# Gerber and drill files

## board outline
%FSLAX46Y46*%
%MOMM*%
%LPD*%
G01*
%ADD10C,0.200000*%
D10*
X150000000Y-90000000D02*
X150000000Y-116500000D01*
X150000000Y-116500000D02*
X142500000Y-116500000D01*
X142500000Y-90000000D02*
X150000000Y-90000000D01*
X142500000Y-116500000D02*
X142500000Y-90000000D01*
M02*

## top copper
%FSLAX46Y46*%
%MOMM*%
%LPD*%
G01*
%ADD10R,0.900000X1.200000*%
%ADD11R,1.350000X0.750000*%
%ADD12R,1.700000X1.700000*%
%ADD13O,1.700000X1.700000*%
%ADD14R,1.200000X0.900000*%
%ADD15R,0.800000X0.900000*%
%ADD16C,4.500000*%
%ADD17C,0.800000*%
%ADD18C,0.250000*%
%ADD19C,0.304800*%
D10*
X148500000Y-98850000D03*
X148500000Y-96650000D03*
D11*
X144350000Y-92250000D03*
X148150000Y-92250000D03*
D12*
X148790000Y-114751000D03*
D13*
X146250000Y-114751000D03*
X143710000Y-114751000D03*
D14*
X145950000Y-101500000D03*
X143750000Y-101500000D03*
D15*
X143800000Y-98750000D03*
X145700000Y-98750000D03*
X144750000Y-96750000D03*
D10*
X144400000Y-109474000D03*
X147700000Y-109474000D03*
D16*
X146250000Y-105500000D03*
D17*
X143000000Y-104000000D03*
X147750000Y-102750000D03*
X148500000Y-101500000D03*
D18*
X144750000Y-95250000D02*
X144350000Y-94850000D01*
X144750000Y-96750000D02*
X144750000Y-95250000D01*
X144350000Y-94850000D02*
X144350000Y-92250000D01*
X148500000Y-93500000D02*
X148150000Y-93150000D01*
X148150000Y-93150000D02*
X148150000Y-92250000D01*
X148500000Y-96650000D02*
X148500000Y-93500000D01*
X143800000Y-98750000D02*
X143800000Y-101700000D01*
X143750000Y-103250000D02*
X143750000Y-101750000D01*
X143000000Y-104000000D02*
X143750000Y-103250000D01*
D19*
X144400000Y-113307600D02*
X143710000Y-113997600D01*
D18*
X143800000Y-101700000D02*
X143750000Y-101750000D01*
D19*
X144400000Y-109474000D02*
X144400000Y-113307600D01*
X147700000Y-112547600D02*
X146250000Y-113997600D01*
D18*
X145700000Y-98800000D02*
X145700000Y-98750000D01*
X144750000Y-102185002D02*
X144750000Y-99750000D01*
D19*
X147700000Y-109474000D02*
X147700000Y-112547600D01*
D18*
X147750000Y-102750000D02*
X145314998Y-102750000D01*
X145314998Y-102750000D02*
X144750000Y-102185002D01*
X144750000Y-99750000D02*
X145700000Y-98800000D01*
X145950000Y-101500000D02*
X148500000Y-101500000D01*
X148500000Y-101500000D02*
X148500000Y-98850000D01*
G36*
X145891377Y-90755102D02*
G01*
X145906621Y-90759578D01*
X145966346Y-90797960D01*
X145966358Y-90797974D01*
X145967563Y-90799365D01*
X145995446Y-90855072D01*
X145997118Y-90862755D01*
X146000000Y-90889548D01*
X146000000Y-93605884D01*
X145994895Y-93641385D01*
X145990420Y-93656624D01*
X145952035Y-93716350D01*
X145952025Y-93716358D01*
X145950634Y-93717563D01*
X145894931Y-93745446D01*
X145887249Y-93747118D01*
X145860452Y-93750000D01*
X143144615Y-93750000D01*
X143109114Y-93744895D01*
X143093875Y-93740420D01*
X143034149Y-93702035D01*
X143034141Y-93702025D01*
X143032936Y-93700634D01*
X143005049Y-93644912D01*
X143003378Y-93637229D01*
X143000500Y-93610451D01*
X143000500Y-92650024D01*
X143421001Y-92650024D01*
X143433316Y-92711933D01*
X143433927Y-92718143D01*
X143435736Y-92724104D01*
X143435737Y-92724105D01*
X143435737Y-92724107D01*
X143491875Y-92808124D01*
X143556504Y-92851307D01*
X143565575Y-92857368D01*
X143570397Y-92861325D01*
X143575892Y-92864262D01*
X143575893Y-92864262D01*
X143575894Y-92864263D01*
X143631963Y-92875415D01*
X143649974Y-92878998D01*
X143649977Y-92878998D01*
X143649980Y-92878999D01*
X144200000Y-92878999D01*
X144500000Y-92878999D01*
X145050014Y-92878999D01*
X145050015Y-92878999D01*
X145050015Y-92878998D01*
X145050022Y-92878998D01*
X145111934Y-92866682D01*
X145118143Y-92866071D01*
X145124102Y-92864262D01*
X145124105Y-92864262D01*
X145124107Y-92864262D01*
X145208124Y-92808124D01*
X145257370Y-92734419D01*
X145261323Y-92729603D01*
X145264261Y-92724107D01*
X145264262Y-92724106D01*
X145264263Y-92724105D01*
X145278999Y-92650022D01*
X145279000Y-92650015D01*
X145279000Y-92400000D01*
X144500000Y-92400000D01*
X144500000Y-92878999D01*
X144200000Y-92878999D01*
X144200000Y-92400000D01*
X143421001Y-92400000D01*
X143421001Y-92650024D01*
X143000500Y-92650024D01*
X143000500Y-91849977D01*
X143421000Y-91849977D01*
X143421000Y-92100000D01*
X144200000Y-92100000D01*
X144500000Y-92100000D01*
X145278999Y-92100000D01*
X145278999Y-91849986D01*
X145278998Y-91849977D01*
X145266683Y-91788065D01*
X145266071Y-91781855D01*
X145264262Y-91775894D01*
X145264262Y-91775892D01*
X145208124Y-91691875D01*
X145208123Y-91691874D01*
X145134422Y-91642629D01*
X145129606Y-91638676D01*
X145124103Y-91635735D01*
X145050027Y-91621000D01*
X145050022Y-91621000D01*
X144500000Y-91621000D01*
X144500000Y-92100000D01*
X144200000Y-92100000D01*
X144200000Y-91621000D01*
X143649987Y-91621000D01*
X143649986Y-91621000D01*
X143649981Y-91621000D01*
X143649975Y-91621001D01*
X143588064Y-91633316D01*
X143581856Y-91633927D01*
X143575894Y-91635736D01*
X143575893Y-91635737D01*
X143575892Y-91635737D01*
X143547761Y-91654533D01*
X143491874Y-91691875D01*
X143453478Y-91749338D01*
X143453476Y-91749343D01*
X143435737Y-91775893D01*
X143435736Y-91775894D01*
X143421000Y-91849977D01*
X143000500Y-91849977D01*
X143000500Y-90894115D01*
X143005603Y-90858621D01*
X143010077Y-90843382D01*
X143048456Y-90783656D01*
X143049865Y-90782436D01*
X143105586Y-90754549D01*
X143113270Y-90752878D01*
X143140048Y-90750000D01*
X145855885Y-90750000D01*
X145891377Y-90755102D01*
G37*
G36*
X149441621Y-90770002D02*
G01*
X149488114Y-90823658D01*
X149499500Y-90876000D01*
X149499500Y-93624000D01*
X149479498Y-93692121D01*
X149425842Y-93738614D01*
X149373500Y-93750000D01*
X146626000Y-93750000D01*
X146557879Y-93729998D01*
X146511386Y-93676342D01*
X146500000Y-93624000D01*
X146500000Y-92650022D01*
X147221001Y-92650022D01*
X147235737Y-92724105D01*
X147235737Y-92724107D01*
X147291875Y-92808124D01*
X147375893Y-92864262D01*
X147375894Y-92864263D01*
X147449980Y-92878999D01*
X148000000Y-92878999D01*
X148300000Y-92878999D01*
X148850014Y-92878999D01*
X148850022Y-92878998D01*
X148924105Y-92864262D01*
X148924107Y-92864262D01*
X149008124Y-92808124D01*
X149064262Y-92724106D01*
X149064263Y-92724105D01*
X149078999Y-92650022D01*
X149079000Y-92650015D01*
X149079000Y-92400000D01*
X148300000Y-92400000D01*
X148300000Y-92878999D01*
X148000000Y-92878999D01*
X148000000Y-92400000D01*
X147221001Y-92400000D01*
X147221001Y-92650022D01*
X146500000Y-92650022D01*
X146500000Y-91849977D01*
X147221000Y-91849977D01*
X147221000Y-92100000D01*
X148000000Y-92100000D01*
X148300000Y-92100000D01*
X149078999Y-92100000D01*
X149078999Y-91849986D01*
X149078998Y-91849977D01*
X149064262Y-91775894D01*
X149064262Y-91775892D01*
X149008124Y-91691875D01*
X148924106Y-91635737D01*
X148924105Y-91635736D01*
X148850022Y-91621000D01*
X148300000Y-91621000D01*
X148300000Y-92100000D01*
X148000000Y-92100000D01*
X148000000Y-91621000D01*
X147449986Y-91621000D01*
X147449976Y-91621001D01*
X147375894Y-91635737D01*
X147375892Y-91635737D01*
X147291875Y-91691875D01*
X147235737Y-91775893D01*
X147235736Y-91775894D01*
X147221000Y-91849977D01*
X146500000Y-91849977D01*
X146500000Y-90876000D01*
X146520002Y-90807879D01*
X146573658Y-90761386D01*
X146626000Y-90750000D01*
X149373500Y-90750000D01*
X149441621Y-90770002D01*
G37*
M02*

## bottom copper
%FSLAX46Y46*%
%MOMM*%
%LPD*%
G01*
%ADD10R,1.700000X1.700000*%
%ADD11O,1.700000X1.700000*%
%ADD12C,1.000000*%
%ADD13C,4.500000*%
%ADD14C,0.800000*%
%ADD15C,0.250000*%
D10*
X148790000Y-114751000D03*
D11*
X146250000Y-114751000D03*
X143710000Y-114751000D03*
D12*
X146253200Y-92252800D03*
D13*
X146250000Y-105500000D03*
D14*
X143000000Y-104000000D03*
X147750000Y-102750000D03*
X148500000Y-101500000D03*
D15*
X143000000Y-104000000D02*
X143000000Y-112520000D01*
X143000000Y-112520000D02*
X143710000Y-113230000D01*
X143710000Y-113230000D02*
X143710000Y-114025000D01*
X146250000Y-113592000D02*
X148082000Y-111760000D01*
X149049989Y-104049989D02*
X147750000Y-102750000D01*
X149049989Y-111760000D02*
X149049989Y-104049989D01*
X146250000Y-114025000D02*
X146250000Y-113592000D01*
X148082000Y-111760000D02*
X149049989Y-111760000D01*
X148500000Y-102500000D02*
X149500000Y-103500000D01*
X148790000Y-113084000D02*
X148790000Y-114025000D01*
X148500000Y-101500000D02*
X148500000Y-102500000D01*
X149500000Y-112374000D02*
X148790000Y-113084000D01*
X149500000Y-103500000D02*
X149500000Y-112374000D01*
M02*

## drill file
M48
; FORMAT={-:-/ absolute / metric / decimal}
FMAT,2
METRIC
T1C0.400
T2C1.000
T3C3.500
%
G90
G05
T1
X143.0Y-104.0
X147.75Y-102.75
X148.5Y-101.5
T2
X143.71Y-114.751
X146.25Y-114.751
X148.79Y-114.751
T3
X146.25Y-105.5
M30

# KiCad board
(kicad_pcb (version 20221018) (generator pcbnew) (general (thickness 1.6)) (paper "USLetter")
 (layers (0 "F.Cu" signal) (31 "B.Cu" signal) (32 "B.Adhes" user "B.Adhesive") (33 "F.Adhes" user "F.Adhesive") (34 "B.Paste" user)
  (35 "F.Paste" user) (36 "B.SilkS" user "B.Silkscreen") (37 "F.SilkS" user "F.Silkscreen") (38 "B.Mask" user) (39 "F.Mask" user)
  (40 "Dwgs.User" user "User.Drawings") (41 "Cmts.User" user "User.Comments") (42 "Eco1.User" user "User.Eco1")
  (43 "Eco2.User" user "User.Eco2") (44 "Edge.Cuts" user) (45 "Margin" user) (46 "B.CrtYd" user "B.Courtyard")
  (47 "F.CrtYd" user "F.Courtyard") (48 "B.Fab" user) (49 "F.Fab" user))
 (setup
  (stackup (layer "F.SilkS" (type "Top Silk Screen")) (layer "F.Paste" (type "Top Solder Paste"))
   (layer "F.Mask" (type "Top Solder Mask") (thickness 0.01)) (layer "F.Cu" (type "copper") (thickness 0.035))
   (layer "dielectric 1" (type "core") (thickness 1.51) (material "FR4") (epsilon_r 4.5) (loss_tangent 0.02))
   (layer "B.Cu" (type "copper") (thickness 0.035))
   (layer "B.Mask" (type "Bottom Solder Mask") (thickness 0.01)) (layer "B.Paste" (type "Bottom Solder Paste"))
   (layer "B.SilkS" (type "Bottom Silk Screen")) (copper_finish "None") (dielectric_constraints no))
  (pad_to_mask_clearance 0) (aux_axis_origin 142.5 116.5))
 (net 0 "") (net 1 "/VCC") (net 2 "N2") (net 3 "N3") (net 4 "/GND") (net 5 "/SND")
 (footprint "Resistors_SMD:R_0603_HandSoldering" (layer "F.Cu") (at 148.5 97.75 90)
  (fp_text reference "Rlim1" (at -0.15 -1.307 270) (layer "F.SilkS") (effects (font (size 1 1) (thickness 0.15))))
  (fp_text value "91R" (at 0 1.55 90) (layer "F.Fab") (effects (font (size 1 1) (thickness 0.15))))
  (pad "1" smd rect (at -1.1 0 90) (size 1.2 0.9) (layers "F.Cu" "F.Paste" "F.Mask") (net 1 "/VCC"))
  (pad "2" smd rect (at 1.1 0 90) (size 1.2 0.9) (layers "F.Cu" "F.Paste" "F.Mask") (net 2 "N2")))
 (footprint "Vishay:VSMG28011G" (layer "F.Cu") (at 146.25 92.25)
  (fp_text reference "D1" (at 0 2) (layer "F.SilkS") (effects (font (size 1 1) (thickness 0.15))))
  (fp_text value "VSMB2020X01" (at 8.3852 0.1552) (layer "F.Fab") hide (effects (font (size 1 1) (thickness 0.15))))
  (pad "1" smd rect (at -1.9 0) (size 1.35 0.75) (layers "F.Cu" "F.Paste" "F.Mask") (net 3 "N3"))
  (pad "2" smd rect (at 1.9 0) (size 1.35 0.75) (layers "F.Cu" "F.Paste" "F.Mask") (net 2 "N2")))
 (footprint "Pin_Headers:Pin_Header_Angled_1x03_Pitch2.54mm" (layer "F.Cu") (at 148.79 114.751 -90)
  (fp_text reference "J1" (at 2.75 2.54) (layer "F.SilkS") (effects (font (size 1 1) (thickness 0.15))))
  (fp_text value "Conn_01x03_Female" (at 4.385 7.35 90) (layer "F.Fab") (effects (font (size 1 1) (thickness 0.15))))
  (pad "1" thru_hole rect (at 0 0 270) (size 1.7 1.7) (drill 1) (layers "*.Cu" "*.Mask") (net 1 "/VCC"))
  (pad "2" thru_hole oval (at 0 2.54 270) (size 1.7 1.7) (drill 1) (layers "*.Cu" "*.Mask") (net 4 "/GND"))
  (pad "3" thru_hole oval (at 0 5.08 270) (size 1.7 1.7) (drill 1) (layers "*.Cu" "*.Mask") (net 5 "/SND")))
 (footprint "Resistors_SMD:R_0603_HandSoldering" (layer "F.Cu") (at 144.85 101.5 180)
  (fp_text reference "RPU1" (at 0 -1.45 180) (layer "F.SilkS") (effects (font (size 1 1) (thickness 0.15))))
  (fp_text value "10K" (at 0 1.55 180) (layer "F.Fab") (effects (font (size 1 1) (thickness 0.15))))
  (pad "1" smd rect (at -1.1 0 180) (size 1.2 0.9) (layers "F.Cu" "F.Paste" "F.Mask") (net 1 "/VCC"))
  (pad "2" smd rect (at 1.1 0 180) (size 1.2 0.9) (layers "F.Cu" "F.Paste" "F.Mask") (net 5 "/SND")))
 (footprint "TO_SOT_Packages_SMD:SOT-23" (layer "F.Cu") (at 144.75 97.75 90)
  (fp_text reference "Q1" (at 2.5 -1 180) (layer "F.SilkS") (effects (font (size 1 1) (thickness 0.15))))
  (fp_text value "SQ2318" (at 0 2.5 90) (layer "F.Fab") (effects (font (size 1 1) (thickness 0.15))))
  (pad "1" smd rect (at -1 -0.95 90) (size 0.9 0.8) (layers "F.Cu" "F.Paste" "F.Mask") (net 5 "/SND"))
  (pad "2" smd rect (at -1 0.95 90) (size 0.9 0.8) (layers "F.Cu" "F.Paste" "F.Mask") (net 4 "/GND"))
  (pad "3" smd rect (at 1 0 90) (size 0.9 0.8) (layers "F.Cu" "F.Paste" "F.Mask") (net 3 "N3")))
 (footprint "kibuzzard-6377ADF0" (layer "F.Cu") (at 147.574 112.395 90)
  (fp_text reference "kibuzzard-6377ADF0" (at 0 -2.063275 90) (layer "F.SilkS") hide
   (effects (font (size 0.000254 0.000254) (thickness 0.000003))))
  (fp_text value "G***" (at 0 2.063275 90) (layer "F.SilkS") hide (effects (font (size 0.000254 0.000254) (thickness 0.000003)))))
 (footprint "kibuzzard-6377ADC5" (layer "F.Cu") (at 144.018 112.014 90)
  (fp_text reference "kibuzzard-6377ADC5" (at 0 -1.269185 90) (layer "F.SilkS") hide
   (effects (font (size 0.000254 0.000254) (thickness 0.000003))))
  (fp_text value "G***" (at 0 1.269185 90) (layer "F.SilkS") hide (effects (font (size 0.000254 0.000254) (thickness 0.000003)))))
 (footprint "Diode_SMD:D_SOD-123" (layer "F.Cu") (at 146.05 109.474)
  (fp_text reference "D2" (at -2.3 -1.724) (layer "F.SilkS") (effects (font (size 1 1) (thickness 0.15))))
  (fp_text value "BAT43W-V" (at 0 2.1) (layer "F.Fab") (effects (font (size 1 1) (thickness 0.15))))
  (pad "1" smd rect (at -1.65 0) (size 0.9 1.2) (layers "F.Cu" "F.Paste" "F.Mask") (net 5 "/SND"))
  (pad "2" smd rect (at 1.65 0) (size 0.9 1.2) (layers "F.Cu" "F.Paste" "F.Mask") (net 4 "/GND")))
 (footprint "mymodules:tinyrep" (layer "B.Cu") (at 148.717 97.663 90)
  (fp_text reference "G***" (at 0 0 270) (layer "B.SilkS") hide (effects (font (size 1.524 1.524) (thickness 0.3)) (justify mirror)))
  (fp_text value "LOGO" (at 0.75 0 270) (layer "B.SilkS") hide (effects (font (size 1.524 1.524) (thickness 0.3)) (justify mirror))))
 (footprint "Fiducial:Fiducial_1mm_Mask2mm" (layer "B.Cu") (at 146.2532 92.2528 180)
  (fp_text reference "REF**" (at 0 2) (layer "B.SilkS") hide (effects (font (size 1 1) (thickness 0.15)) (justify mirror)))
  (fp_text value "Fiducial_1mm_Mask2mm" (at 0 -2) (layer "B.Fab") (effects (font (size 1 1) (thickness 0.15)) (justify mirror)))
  (pad "" smd circle (at 0 0 180) (size 1 1) (layers "B.Cu" "B.Mask") (solder_mask_margin 0.5) (clearance 0.5)))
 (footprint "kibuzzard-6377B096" (layer "B.Cu") (at 147.574 112.395 -90)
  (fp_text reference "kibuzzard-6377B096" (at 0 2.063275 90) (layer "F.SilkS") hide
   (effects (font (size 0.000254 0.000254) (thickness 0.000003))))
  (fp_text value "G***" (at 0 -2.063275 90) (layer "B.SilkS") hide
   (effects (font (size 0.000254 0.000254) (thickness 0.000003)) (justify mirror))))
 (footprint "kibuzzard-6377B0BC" (layer "B.Cu") (at 144.018 112.014 90)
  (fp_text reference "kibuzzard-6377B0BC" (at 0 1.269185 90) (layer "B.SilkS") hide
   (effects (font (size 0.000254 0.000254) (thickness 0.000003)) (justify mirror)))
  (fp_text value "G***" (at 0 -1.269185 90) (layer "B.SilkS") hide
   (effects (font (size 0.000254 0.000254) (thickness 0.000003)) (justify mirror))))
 (gr_line (start 150 90) (end 150 116.5) (stroke (width 0.2) (type solid)) (layer "Edge.Cuts"))
 (gr_line (start 150 116.5) (end 142.5 116.5) (stroke (width 0.2) (type solid)) (layer "Edge.Cuts"))
 (gr_line (start 142.5 90) (end 150 90) (stroke (width 0.2) (type solid)) (layer "Edge.Cuts"))
 (gr_line (start 142.5 116.5) (end 142.5 90) (stroke (width 0.2) (type solid)) (layer "Edge.Cuts"))
 (via (at 146.25 105.5) (size 4.5) (drill 3.5) (layers "F.Cu" "B.Cu") (free) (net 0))
 (segment (start 144.75 95.25) (end 144.35 94.85) (width 0.25) (layer "F.Cu") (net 3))
 (segment (start 144.75 96.75) (end 144.75 95.25) (width 0.25) (layer "F.Cu") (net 3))
 (segment (start 144.35 94.85) (end 144.35 92.25) (width 0.25) (layer "F.Cu") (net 3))
 (segment (start 148.5 93.5) (end 148.15 93.15) (width 0.25) (layer "F.Cu") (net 2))
 (segment (start 148.15 93.15) (end 148.15 92.25) (width 0.25) (layer "F.Cu") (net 2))
 (segment (start 148.5 96.65) (end 148.5 93.5) (width 0.25) (layer "F.Cu") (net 2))
 (segment (start 143.8 98.75) (end 143.8 101.7) (width 0.25) (layer "F.Cu") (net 5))
 (segment (start 143.75 103.25) (end 143.75 101.75) (width 0.25) (layer "F.Cu") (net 5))
 (segment (start 143 104) (end 143.75 103.25) (width 0.25) (layer "F.Cu") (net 5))
 (segment (start 144.4 113.3076) (end 143.71 113.9976) (width 0.3048) (layer "F.Cu") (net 5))
 (segment (start 143.8 101.7) (end 143.75 101.75) (width 0.25) (layer "F.Cu") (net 5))
 (segment (start 144.4 109.474) (end 144.4 113.3076) (width 0.3048) (layer "F.Cu") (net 5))
 (via (at 143 104) (size 0.8) (drill 0.4) (layers "F.Cu" "B.Cu") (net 5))
 (segment (start 143 104) (end 143 112.52) (width 0.25) (layer "B.Cu") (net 5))
 (segment (start 143 112.52) (end 143.71 113.23) (width 0.25) (layer "B.Cu") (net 5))
 (segment (start 143.71 113.23) (end 143.71 114.025) (width 0.25) (layer "B.Cu") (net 5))
 (segment (start 147.7 112.5476) (end 146.25 113.9976) (width 0.3048) (layer "F.Cu") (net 4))
 (segment (start 145.7 98.8) (end 145.7 98.75) (width 0.25) (layer "F.Cu") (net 4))
 (segment (start 144.75 102.185002) (end 144.75 99.75) (width 0.25) (layer "F.Cu") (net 4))
 (segment (start 147.7 109.474) (end 147.7 112.5476) (width 0.3048) (layer "F.Cu") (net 4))
 (segment (start 147.75 102.75) (end 145.314998 102.75) (width 0.25) (layer "F.Cu") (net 4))
 (segment (start 145.314998 102.75) (end 144.75 102.185002) (width 0.25) (layer "F.Cu") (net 4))
 (segment (start 144.75 99.75) (end 145.7 98.8) (width 0.25) (layer "F.Cu") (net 4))
 (via (at 147.75 102.75) (size 0.8) (drill 0.4) (layers "F.Cu" "B.Cu") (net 4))
 (segment (start 146.25 113.592) (end 148.082 111.76) (width 0.25) (layer "B.Cu") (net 4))
 (segment (start 149.049989 104.049989) (end 147.75 102.75) (width 0.25) (layer "B.Cu") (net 4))
 (segment (start 149.049989 111.76) (end 149.049989 104.049989) (width 0.25) (layer "B.Cu") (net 4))
 (segment (start 146.25 114.025) (end 146.25 113.592) (width 0.25) (layer "B.Cu") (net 4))
 (segment (start 148.082 111.76) (end 149.049989 111.76) (width 0.25) (layer "B.Cu") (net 4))
 (segment (start 145.95 101.5) (end 148.5 101.5) (width 0.25) (layer "F.Cu") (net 1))
 (segment (start 148.5 101.5) (end 148.5 98.85) (width 0.25) (layer "F.Cu") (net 1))
 (via (at 148.5 101.5) (size 0.8) (drill 0.4) (layers "F.Cu" "B.Cu") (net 1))
 (segment (start 148.5 102.5) (end 149.5 103.5) (width 0.25) (layer "B.Cu") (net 1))
 (segment (start 148.79 113.084) (end 148.79 114.025) (width 0.25) (layer "B.Cu") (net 1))
 (segment (start 148.5 101.5) (end 148.5 102.5) (width 0.25) (layer "B.Cu") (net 1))
 (segment (start 149.5 112.374) (end 148.79 113.084) (width 0.25) (layer "B.Cu") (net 1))
 (segment (start 149.5 103.5) (end 149.5 112.374) (width 0.25) (layer "B.Cu") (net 1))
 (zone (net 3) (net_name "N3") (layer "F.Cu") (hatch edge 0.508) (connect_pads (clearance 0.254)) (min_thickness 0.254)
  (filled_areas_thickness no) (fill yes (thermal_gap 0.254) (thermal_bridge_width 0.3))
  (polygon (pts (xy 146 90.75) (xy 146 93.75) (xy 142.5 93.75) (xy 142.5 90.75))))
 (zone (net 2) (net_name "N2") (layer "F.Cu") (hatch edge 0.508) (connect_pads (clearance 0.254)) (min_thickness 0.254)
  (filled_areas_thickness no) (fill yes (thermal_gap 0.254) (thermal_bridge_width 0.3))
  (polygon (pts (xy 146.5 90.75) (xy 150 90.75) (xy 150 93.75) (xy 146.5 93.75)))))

